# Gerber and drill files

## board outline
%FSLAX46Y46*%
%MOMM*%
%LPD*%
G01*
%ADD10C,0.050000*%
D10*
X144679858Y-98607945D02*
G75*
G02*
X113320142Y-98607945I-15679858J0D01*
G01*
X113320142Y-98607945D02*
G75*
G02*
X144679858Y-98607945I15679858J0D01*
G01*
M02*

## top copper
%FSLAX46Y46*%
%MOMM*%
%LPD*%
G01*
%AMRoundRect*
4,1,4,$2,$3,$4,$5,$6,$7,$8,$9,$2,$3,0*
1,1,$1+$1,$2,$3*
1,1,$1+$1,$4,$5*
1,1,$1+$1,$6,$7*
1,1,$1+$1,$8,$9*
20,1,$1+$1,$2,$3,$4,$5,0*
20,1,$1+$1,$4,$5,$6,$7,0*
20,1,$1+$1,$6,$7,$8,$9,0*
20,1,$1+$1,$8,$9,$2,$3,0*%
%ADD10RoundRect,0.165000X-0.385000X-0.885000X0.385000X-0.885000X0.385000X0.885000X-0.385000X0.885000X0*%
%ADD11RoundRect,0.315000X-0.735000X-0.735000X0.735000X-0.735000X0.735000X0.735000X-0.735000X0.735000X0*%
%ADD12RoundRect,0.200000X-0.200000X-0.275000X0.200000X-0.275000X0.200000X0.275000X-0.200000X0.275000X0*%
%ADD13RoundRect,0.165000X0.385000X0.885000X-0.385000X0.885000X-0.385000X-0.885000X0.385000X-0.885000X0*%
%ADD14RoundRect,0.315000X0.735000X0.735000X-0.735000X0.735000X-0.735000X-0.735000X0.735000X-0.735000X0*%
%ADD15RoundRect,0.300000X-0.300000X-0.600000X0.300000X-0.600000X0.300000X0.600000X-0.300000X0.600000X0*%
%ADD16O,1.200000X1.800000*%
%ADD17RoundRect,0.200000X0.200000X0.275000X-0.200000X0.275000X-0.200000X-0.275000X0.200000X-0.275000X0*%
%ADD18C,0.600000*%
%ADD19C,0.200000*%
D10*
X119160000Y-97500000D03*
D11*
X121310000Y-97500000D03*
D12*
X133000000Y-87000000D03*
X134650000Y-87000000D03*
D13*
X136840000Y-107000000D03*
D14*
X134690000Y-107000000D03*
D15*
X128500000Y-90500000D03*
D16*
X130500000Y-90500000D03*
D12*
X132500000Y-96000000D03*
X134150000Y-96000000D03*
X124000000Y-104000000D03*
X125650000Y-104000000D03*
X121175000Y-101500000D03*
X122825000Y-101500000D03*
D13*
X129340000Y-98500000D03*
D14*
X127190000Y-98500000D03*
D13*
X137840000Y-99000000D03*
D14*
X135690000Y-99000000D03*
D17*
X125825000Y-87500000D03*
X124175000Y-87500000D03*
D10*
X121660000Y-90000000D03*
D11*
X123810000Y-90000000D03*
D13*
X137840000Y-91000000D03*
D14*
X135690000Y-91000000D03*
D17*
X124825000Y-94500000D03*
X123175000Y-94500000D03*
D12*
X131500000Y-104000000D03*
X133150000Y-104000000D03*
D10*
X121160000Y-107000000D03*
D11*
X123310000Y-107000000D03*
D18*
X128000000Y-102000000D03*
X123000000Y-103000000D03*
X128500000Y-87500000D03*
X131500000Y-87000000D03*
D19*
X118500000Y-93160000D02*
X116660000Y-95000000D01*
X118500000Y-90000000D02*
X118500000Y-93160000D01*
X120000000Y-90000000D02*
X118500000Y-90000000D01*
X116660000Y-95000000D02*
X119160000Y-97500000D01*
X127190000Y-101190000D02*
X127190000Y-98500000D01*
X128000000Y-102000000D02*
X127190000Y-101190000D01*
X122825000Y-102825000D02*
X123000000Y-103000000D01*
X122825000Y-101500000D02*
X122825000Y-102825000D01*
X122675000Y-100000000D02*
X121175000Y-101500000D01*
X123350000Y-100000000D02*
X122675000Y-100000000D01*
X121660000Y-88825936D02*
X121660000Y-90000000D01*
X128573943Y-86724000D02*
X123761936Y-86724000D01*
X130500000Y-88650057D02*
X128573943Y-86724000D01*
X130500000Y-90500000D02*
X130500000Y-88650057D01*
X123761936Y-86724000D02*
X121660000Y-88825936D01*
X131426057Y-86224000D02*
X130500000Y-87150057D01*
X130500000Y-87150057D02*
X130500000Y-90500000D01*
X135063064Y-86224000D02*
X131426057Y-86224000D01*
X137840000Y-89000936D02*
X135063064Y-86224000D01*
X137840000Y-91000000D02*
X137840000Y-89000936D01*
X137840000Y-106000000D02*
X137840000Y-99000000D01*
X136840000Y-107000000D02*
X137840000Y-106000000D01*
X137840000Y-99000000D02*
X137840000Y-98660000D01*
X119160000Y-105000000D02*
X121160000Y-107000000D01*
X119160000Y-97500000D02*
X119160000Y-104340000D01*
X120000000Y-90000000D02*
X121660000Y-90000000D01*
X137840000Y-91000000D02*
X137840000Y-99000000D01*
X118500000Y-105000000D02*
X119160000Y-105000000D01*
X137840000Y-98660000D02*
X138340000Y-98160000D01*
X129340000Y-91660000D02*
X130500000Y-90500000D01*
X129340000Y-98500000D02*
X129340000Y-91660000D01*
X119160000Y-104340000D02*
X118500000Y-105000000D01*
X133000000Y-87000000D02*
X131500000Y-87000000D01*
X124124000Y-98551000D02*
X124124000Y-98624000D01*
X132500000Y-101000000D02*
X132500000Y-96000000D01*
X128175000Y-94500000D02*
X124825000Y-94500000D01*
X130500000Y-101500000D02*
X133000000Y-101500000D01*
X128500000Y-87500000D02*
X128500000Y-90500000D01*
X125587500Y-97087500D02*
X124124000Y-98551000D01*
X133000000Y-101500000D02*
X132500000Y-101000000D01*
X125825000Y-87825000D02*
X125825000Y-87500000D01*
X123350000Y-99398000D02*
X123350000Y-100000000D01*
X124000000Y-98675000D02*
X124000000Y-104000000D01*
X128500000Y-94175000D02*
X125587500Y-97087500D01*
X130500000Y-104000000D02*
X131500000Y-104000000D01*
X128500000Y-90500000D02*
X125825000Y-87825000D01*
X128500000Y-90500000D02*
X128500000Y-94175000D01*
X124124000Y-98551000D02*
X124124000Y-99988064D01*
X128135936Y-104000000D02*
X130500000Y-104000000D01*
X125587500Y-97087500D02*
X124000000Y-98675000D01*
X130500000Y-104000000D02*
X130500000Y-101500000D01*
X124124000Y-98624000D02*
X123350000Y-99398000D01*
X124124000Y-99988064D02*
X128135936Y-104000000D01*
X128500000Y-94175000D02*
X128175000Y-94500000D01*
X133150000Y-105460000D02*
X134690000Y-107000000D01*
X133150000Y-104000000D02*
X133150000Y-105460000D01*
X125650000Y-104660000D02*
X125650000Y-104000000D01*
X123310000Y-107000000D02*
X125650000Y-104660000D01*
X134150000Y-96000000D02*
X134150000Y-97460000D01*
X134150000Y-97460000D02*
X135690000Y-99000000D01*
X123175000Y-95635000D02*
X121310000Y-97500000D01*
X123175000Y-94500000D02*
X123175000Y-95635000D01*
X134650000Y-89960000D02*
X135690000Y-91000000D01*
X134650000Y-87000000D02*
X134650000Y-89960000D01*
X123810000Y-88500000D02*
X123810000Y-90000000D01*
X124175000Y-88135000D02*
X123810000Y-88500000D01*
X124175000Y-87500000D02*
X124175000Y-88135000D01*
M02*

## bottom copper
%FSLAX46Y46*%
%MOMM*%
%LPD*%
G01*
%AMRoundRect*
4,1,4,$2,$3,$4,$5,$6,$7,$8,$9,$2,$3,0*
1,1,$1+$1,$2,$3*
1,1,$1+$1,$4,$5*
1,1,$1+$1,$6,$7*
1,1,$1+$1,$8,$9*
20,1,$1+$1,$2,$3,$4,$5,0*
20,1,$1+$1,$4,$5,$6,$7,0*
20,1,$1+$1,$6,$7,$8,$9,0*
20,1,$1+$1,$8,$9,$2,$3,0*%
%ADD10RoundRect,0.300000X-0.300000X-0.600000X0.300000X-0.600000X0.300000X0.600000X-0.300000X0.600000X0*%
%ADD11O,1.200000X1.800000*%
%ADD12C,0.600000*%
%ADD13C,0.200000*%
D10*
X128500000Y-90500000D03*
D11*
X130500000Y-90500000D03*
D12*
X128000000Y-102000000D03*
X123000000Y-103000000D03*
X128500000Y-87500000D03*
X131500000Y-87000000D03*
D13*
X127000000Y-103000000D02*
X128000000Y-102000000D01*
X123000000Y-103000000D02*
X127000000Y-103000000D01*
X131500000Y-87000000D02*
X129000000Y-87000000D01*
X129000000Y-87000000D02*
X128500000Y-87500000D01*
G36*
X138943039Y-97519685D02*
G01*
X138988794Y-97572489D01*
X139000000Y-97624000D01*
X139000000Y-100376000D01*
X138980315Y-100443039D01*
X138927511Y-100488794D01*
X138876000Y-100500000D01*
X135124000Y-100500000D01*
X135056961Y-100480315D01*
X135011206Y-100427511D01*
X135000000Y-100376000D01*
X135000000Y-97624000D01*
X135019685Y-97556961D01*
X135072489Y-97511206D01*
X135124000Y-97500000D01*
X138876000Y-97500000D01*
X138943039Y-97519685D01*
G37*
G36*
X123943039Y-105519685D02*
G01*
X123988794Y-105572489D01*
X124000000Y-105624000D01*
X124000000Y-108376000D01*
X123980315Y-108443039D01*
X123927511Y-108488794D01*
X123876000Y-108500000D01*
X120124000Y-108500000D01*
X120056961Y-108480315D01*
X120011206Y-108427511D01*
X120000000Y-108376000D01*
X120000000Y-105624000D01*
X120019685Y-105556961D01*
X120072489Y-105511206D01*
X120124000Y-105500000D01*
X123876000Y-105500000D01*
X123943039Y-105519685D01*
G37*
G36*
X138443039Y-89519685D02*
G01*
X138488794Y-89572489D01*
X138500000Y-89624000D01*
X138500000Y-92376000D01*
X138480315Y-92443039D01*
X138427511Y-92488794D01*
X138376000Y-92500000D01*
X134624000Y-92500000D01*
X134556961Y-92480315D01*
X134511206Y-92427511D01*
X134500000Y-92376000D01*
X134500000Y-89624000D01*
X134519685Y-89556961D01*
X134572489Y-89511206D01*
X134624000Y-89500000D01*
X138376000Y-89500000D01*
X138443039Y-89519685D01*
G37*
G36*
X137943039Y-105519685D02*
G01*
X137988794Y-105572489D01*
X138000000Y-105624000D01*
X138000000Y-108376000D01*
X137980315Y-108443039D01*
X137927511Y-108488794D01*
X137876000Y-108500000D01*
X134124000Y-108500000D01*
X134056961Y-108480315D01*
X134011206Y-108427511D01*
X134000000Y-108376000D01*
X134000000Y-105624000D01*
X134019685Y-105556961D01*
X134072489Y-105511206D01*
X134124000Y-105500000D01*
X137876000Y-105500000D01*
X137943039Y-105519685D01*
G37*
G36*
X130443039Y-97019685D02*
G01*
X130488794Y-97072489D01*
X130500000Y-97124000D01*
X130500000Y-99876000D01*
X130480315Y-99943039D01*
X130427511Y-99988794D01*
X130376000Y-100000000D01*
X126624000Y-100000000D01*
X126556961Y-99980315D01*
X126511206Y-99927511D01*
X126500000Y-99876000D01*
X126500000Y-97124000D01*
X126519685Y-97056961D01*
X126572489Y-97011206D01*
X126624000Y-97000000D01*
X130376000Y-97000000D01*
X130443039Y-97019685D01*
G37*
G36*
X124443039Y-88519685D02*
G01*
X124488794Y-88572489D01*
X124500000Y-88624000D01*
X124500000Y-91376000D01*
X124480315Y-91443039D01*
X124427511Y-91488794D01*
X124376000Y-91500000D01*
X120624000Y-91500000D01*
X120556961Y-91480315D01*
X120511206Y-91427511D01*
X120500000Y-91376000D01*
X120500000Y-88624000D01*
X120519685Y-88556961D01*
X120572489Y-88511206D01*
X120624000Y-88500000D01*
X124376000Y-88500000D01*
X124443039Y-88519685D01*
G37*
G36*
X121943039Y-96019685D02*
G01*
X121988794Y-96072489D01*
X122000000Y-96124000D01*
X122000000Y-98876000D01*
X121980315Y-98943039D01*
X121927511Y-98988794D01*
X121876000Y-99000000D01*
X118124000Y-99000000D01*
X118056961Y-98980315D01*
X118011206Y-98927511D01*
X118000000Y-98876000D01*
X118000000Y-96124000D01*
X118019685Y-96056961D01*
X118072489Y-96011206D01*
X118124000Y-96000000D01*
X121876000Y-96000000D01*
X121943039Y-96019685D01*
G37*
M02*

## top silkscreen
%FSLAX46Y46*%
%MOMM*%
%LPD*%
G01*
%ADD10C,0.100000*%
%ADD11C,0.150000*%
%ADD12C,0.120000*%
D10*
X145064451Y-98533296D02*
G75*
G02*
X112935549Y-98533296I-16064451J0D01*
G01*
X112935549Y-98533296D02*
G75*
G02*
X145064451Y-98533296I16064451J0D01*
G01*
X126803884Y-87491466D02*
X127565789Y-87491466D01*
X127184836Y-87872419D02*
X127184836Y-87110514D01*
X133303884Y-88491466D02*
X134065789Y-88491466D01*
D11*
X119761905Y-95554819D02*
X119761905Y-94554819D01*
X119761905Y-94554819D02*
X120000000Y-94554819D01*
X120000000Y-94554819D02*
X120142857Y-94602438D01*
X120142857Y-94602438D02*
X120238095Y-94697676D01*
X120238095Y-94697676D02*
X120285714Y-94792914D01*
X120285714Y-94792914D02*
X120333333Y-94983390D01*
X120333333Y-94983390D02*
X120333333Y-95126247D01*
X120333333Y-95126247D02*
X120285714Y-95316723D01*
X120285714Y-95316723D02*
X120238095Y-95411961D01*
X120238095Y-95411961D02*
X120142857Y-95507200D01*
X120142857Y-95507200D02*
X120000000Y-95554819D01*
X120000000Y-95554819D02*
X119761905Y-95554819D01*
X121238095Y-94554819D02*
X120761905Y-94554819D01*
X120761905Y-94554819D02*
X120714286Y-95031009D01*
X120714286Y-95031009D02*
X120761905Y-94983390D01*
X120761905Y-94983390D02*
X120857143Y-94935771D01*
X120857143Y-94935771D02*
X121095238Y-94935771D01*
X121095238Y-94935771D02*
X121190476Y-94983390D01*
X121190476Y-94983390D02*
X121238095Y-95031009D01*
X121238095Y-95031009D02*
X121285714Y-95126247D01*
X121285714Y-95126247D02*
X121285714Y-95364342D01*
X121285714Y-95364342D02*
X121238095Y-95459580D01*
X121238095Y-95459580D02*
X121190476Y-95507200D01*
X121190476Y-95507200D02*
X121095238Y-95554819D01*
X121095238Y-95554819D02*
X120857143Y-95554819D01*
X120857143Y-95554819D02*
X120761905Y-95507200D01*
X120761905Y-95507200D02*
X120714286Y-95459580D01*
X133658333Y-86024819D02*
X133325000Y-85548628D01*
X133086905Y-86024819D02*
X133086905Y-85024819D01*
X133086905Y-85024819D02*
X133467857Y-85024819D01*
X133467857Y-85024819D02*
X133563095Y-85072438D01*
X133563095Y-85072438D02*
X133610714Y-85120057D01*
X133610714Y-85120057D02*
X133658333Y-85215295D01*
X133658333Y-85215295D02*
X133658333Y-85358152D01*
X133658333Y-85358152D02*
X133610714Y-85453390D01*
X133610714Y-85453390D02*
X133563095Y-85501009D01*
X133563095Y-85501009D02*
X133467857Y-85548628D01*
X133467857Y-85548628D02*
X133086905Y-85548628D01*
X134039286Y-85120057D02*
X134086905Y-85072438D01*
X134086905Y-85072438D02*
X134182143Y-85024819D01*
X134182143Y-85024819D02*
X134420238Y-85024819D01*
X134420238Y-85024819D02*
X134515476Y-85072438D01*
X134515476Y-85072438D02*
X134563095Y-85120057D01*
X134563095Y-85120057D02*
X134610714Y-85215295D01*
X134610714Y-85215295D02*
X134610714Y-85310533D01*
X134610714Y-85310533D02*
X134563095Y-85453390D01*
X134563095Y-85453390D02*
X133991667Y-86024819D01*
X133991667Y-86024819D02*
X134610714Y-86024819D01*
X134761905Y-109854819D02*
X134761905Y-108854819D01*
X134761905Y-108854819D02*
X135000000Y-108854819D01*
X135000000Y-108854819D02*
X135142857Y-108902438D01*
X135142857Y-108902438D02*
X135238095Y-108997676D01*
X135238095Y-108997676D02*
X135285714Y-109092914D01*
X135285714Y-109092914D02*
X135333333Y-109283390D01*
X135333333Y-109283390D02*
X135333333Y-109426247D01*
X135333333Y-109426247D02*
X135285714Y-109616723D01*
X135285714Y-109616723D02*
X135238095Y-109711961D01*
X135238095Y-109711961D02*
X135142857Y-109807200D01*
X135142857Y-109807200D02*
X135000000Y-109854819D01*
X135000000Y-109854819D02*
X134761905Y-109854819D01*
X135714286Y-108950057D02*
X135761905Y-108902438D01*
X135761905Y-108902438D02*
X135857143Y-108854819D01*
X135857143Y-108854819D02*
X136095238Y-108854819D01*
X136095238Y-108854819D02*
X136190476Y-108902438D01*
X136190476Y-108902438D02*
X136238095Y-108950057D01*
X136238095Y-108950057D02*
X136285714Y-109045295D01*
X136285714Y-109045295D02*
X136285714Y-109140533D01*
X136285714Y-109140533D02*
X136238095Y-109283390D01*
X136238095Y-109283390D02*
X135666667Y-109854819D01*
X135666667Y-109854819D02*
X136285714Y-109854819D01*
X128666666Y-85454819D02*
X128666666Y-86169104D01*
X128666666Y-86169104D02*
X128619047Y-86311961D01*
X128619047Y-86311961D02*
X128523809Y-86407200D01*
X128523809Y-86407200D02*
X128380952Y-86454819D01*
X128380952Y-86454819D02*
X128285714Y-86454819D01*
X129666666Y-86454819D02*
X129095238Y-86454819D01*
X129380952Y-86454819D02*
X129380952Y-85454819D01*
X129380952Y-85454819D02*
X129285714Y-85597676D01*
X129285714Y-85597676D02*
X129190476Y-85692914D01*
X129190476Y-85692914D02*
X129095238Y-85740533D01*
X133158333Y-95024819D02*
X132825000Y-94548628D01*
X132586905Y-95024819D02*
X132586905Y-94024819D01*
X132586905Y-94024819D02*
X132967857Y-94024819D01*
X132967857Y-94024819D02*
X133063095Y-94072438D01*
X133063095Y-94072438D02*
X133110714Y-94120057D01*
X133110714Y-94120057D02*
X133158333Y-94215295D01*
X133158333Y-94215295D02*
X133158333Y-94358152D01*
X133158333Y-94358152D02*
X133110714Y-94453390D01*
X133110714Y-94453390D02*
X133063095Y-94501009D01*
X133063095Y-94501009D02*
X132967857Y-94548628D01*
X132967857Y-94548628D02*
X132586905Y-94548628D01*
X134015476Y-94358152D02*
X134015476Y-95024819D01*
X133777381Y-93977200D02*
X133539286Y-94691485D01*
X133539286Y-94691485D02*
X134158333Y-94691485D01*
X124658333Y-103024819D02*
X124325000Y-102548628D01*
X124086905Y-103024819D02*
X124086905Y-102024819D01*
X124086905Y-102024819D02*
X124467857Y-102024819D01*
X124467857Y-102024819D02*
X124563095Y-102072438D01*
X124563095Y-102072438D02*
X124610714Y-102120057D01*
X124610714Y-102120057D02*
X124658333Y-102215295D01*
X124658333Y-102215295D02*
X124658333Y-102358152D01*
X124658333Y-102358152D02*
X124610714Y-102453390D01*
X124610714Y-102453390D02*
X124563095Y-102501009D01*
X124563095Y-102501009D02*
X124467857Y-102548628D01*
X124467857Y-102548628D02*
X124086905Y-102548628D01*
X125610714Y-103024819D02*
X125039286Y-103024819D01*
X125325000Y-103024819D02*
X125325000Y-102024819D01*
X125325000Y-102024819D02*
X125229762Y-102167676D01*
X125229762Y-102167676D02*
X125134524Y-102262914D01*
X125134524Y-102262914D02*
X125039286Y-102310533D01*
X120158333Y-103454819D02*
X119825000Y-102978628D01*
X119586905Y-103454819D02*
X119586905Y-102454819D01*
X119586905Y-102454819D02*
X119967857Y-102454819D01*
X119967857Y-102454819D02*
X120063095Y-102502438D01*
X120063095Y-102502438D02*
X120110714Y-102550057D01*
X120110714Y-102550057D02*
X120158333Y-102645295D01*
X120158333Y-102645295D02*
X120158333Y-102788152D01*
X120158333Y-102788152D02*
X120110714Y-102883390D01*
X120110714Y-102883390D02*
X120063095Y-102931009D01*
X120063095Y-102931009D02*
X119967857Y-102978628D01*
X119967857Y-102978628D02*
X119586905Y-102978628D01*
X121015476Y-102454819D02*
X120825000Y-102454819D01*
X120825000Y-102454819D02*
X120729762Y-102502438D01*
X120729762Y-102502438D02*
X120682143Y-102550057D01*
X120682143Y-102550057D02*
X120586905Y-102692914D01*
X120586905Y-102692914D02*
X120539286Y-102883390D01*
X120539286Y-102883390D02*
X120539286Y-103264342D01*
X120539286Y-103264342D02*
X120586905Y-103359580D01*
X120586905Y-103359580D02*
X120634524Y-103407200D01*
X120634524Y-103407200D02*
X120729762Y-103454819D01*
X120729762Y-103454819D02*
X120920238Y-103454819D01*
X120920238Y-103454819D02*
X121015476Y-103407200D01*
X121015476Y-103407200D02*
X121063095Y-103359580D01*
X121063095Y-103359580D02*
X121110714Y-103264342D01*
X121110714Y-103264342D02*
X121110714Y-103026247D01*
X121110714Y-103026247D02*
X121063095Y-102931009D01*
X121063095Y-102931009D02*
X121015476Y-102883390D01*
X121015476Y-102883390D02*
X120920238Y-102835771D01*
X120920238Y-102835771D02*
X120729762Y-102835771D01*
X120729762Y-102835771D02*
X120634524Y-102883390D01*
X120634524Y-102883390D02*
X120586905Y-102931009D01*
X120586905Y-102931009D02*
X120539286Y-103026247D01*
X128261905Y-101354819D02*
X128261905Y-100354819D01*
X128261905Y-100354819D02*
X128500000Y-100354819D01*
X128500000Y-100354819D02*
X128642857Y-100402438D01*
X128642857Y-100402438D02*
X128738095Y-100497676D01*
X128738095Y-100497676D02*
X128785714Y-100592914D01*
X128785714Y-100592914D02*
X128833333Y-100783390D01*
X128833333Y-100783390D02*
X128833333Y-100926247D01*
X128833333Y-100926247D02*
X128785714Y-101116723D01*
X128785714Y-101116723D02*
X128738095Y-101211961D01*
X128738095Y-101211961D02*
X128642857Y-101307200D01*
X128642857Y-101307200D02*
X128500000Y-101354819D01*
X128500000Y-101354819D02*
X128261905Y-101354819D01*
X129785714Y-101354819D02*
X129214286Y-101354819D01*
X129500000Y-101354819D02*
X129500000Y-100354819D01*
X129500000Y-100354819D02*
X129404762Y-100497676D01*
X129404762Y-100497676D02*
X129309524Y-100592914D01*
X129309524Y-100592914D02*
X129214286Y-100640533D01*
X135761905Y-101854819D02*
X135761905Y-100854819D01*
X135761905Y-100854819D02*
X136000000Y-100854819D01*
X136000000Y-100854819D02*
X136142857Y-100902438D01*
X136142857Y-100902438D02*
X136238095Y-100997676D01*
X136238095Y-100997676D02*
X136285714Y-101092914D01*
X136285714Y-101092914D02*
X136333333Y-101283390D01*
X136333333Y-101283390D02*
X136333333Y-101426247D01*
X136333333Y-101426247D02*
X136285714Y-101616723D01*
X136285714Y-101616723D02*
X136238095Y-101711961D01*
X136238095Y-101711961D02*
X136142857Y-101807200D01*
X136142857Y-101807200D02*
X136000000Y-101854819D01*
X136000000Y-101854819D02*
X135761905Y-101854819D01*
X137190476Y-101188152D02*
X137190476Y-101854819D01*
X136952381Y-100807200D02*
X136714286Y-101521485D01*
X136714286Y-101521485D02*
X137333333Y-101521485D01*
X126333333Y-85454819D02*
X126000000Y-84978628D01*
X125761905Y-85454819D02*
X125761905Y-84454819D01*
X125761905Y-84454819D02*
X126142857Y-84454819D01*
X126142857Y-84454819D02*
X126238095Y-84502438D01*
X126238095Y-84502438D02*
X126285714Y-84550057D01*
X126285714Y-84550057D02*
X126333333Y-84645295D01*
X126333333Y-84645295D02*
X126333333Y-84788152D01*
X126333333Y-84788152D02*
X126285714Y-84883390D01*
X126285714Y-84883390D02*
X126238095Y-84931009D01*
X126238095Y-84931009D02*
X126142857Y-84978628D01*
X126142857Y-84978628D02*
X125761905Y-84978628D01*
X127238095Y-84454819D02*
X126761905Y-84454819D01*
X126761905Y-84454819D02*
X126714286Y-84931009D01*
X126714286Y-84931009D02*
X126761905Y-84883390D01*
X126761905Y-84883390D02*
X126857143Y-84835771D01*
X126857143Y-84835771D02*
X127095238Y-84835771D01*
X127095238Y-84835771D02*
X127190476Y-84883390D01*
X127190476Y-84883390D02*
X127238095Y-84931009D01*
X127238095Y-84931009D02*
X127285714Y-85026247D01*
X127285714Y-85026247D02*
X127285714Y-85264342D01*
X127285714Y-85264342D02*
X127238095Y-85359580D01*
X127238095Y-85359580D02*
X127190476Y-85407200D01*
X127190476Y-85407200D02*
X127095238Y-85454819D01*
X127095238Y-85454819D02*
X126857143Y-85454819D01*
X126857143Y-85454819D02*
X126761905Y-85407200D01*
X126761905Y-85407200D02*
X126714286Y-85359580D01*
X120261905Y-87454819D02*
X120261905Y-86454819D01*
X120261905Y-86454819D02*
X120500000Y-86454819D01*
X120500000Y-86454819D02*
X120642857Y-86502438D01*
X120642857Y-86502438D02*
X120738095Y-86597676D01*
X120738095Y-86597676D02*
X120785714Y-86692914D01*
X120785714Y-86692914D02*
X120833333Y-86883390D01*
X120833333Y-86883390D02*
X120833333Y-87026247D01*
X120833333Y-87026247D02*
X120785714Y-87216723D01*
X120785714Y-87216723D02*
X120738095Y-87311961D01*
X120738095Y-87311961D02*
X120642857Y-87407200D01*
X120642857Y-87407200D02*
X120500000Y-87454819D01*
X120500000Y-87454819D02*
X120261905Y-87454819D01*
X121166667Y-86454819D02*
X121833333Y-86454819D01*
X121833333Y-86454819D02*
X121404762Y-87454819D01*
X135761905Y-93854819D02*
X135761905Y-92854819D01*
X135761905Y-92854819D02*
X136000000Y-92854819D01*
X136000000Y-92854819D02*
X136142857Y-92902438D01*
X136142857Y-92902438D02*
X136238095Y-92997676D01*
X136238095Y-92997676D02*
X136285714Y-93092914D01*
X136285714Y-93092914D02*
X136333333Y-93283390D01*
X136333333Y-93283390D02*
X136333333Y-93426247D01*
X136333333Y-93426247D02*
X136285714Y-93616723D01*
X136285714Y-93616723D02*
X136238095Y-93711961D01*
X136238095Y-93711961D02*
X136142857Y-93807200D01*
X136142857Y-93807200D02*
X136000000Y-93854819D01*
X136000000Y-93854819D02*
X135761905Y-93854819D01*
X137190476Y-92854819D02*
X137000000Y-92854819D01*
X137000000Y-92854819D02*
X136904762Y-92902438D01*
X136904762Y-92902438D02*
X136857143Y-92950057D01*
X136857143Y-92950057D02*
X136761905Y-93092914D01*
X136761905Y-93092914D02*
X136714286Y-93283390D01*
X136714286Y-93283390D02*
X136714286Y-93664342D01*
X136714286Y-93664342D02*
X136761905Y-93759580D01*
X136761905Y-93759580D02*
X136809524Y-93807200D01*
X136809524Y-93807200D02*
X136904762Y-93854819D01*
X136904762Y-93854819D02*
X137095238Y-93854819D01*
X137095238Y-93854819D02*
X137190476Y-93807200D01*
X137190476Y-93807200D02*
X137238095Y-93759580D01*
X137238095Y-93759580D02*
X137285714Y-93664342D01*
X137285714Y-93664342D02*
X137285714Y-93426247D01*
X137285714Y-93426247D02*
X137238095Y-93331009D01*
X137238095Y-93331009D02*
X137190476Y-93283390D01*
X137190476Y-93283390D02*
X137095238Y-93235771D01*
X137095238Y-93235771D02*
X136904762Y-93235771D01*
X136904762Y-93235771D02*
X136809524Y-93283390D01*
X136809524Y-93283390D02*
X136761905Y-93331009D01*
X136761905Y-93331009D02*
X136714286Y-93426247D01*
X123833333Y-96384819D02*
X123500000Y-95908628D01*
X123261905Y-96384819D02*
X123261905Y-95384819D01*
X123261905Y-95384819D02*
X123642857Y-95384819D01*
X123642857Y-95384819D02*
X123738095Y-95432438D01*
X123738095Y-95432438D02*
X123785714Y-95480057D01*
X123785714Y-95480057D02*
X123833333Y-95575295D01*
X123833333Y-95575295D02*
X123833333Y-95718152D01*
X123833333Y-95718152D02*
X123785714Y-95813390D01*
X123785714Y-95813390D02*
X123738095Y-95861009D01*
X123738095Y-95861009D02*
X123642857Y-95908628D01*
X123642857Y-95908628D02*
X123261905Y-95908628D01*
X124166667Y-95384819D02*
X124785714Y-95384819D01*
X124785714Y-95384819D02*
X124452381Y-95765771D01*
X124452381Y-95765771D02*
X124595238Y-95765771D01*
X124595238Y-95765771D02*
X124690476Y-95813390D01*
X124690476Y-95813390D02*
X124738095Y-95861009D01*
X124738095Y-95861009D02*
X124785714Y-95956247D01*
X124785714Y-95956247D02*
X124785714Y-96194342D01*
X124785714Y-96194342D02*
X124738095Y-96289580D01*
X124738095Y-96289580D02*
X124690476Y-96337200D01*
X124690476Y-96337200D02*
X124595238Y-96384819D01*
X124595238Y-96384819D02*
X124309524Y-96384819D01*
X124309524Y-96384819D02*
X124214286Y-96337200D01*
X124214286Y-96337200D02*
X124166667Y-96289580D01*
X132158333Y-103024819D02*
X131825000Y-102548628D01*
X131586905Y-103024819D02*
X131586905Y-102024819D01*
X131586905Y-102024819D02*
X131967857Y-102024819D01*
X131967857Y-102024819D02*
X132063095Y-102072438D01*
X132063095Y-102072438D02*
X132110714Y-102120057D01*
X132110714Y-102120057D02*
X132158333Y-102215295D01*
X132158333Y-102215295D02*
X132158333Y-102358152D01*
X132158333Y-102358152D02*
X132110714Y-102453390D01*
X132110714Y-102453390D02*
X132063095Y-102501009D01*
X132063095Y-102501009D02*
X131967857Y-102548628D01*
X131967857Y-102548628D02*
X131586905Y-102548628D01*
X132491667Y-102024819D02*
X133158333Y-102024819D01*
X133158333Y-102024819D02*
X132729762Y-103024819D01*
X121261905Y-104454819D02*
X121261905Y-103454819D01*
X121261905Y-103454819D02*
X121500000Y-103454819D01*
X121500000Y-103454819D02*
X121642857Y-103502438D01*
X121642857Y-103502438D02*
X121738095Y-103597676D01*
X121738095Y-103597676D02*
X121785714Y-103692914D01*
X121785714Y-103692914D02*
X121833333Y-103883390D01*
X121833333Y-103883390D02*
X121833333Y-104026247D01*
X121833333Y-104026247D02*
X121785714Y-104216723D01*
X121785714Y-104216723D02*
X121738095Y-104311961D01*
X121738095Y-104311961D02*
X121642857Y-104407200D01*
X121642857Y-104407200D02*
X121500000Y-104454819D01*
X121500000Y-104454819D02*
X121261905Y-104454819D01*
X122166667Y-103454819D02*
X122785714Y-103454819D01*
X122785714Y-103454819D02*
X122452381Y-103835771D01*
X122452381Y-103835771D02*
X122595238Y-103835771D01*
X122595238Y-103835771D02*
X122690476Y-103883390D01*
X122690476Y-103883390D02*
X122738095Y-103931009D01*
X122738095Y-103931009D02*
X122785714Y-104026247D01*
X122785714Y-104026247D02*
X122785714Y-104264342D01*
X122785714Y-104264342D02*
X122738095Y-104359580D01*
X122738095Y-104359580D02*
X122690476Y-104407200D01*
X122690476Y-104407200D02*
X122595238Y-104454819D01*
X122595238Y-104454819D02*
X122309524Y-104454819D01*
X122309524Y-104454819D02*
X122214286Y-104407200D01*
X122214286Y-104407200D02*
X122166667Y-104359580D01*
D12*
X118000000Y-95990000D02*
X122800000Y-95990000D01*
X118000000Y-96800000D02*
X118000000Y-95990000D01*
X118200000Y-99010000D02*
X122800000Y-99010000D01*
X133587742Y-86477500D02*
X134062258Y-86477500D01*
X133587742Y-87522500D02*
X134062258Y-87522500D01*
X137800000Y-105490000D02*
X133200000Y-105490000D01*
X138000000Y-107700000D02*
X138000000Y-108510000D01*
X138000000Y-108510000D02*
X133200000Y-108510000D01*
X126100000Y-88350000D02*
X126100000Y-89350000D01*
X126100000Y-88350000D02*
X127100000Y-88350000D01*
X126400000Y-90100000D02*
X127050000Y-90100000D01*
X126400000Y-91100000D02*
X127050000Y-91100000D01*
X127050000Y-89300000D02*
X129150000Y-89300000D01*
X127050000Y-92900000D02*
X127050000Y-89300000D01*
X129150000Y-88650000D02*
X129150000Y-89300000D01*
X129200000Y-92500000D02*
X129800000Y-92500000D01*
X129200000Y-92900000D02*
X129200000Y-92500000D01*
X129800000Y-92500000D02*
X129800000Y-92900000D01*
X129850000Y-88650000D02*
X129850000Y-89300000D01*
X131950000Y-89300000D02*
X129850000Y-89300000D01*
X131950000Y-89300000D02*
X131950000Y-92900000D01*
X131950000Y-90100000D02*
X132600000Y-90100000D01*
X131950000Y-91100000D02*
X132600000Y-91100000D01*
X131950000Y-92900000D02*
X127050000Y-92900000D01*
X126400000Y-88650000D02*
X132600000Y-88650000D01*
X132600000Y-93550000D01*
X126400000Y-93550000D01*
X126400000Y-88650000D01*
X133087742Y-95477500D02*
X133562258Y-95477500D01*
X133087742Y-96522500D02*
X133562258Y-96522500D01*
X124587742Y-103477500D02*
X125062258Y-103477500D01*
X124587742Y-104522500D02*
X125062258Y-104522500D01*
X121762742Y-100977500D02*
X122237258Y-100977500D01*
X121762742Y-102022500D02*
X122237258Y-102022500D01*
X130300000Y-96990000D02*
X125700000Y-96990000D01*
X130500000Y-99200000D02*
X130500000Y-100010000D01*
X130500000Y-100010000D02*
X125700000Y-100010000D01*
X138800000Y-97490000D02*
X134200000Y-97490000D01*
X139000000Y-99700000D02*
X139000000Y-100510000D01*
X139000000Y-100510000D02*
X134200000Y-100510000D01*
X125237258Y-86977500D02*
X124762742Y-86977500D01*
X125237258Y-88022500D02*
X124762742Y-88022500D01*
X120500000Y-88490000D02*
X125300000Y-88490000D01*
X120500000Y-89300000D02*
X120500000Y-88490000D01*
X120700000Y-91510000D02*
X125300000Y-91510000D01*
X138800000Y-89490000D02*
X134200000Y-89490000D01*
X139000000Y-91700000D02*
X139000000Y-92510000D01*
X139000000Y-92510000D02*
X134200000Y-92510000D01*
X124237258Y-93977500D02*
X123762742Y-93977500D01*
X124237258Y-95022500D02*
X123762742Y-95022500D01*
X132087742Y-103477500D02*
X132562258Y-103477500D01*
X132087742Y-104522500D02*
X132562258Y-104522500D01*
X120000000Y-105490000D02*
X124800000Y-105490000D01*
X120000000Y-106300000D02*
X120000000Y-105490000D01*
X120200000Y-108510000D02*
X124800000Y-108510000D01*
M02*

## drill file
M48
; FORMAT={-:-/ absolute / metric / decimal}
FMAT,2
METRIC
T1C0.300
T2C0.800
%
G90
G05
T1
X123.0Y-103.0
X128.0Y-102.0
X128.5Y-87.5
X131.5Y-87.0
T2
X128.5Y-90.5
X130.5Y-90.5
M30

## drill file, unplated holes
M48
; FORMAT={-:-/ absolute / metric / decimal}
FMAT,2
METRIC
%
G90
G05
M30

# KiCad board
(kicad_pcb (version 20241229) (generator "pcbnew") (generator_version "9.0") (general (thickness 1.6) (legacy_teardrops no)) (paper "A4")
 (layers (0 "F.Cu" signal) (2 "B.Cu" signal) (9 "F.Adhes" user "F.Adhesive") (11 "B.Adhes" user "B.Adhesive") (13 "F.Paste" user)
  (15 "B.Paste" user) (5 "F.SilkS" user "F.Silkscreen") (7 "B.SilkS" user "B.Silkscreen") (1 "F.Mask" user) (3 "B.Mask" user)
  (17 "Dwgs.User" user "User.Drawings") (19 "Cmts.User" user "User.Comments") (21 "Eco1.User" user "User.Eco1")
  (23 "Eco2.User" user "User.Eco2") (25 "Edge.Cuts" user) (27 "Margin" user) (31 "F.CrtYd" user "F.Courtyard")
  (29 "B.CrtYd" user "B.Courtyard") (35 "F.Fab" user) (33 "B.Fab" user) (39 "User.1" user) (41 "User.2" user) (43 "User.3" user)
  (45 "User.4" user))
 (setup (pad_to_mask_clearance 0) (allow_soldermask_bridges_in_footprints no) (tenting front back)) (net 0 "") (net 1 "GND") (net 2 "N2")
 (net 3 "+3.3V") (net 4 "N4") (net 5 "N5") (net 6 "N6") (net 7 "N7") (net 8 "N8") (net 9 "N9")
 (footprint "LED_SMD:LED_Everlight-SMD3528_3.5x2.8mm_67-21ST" (layer "F.Cu") (at 120.5 97.5)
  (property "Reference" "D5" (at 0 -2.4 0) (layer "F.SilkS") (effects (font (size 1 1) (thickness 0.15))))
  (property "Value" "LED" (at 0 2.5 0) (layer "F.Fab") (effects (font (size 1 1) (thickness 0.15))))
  (fp_line (start -2.5 -1.51) (end 2.3 -1.51) (stroke (width 0.12) (type solid)) (layer "F.SilkS"))
  (fp_line (start -2.5 -0.7) (end -2.5 -1.51) (stroke (width 0.12) (type solid)) (layer "F.SilkS"))
  (fp_line (start -2.3 1.51) (end 2.3 1.51) (stroke (width 0.12) (type solid)) (layer "F.SilkS"))
  (pad "1" smd roundrect (at -1.34 0) (size 1.1 2.1) (layers "F.Cu" "F.Mask" "F.Paste") (roundrect_rratio 0.15) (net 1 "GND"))
  (pad "2" smd roundrect (at 0.81 0) (size 2.1 2.1) (layers "F.Cu" "F.Mask" "F.Paste") (roundrect_rratio 0.15) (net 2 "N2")))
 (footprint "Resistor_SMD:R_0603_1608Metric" (layer "F.Cu") (at 133.825 87)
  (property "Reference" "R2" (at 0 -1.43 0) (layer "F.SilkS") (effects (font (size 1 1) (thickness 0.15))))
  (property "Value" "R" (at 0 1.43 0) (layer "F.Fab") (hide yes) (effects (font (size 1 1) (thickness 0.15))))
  (fp_line (start -0.237258 -0.5225) (end 0.237258 -0.5225) (stroke (width 0.12) (type solid)) (layer "F.SilkS"))
  (fp_line (start -0.237258 0.5225) (end 0.237258 0.5225) (stroke (width 0.12) (type solid)) (layer "F.SilkS"))
  (pad "1" smd roundrect (at -0.825 0) (size 0.8 0.95) (layers "F.Cu" "F.Mask" "F.Paste") (roundrect_rratio 0.25) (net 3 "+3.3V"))
  (pad "2" smd roundrect (at 0.825 0) (size 0.8 0.95) (layers "F.Cu" "F.Mask" "F.Paste") (roundrect_rratio 0.25) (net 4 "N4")))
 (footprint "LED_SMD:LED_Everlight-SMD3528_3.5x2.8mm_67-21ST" (layer "F.Cu") (at 135.5 107 180)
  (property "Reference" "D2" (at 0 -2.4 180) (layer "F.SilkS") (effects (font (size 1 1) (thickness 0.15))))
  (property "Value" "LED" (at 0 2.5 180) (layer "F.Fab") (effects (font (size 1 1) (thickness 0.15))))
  (fp_line (start -2.3 1.51) (end 2.3 1.51) (stroke (width 0.12) (type solid)) (layer "F.SilkS"))
  (fp_line (start -2.5 -0.7) (end -2.5 -1.51) (stroke (width 0.12) (type solid)) (layer "F.SilkS"))
  (fp_line (start -2.5 -1.51) (end 2.3 -1.51) (stroke (width 0.12) (type solid)) (layer "F.SilkS"))
  (pad "1" smd roundrect (at -1.34 0 180) (size 1.1 2.1) (layers "F.Cu" "F.Mask" "F.Paste") (roundrect_rratio 0.15) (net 1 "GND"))
  (pad "2" smd roundrect (at 0.81 0 180) (size 2.1 2.1) (layers "F.Cu" "F.Mask" "F.Paste") (roundrect_rratio 0.15) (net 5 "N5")))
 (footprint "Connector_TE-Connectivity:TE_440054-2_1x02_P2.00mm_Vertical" (layer "F.Cu") (at 128.5 90.5)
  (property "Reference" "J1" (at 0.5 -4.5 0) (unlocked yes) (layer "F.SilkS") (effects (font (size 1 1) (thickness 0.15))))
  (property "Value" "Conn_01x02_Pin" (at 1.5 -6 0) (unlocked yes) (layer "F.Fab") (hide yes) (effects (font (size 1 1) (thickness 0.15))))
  (fp_line (start -2.4 -2.15) (end -2.4 -1.15) (stroke (width 0.12) (type solid)) (layer "F.SilkS"))
  (fp_line (start -2.4 -2.15) (end -1.4 -2.15) (stroke (width 0.12) (type solid)) (layer "F.SilkS"))
  (fp_line (start -2.1 -0.4) (end -1.45 -0.4) (stroke (width 0.12) (type solid)) (layer "F.SilkS"))
  (fp_line (start -2.1 0.6) (end -1.45 0.6) (stroke (width 0.12) (type solid)) (layer "F.SilkS"))
  (fp_line (start -1.45 -1.2) (end 0.65 -1.2) (stroke (width 0.12) (type solid)) (layer "F.SilkS"))
  (fp_line (start -1.45 2.4) (end -1.45 -1.2) (stroke (width 0.12) (type solid)) (layer "F.SilkS"))
  (fp_line (start 0.65 -1.85) (end 0.65 -1.2) (stroke (width 0.12) (type solid)) (layer "F.SilkS"))
  (fp_line (start 0.7 2) (end 1.3 2) (stroke (width 0.12) (type solid)) (layer "F.SilkS"))
  (fp_line (start 0.7 2.4) (end 0.7 2) (stroke (width 0.12) (type solid)) (layer "F.SilkS"))
  (fp_line (start 1.3 2) (end 1.3 2.4) (stroke (width 0.12) (type solid)) (layer "F.SilkS"))
  (fp_line (start 1.35 -1.85) (end 1.35 -1.2) (stroke (width 0.12) (type solid)) (layer "F.SilkS"))
  (fp_line (start 3.45 -1.2) (end 1.35 -1.2) (stroke (width 0.12) (type solid)) (layer "F.SilkS"))
  (fp_line (start 3.45 -1.2) (end 3.45 2.4) (stroke (width 0.12) (type solid)) (layer "F.SilkS"))
  (fp_line (start 3.45 -0.4) (end 4.1 -0.4) (stroke (width 0.12) (type solid)) (layer "F.SilkS"))
  (fp_line (start 3.45 0.6) (end 4.1 0.6) (stroke (width 0.12) (type solid)) (layer "F.SilkS"))
  (fp_line (start 3.45 2.4) (end -1.45 2.4) (stroke (width 0.12) (type solid)) (layer "F.SilkS"))
  (fp_rect (start -2.1 -1.85) (end 4.1 3.05) (stroke (width 0.12) (type solid)) (fill no) (layer "F.SilkS"))
  (pad "1" thru_hole roundrect (at 0 0) (size 1.2 1.8) (drill 0.8) (layers "*.Cu" "*.Mask") (remove_unused_layers no)
   (roundrect_rratio 0.25) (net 3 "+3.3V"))
  (pad "2" thru_hole oval (at 2 0) (size 1.2 1.8) (drill 0.8) (layers "*.Cu" "*.Mask") (remove_unused_layers no) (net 1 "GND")))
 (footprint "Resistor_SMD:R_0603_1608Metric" (layer "F.Cu") (at 133.325 96)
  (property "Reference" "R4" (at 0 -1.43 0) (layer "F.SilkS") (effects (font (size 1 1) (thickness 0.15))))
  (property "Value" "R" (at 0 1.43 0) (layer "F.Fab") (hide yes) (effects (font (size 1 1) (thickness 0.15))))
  (fp_line (start -0.237258 -0.5225) (end 0.237258 -0.5225) (stroke (width 0.12) (type solid)) (layer "F.SilkS"))
  (fp_line (start -0.237258 0.5225) (end 0.237258 0.5225) (stroke (width 0.12) (type solid)) (layer "F.SilkS"))
  (pad "1" smd roundrect (at -0.825 0) (size 0.8 0.95) (layers "F.Cu" "F.Mask" "F.Paste") (roundrect_rratio 0.25) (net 3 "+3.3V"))
  (pad "2" smd roundrect (at 0.825 0) (size 0.8 0.95) (layers "F.Cu" "F.Mask" "F.Paste") (roundrect_rratio 0.25) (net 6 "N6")))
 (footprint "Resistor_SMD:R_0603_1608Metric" (layer "F.Cu") (at 124.825 104)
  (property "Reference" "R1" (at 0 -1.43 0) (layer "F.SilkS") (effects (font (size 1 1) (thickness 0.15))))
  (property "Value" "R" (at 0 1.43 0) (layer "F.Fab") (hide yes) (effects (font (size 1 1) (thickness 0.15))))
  (fp_line (start -0.237258 -0.5225) (end 0.237258 -0.5225) (stroke (width 0.12) (type solid)) (layer "F.SilkS"))
  (fp_line (start -0.237258 0.5225) (end 0.237258 0.5225) (stroke (width 0.12) (type solid)) (layer "F.SilkS"))
  (pad "1" smd roundrect (at -0.825 0) (size 0.8 0.95) (layers "F.Cu" "F.Mask" "F.Paste") (roundrect_rratio 0.25) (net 3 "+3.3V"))
  (pad "2" smd roundrect (at 0.825 0) (size 0.8 0.95) (layers "F.Cu" "F.Mask" "F.Paste") (roundrect_rratio 0.25) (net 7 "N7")))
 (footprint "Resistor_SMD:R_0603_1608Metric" (layer "F.Cu") (at 122 101.5)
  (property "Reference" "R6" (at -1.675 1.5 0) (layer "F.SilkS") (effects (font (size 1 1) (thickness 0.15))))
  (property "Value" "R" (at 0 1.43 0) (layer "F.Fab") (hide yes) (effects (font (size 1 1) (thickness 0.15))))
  (fp_line (start -0.237258 -0.5225) (end 0.237258 -0.5225) (stroke (width 0.12) (type solid)) (layer "F.SilkS"))
  (fp_line (start -0.237258 0.5225) (end 0.237258 0.5225) (stroke (width 0.12) (type solid)) (layer "F.SilkS"))
  (pad "1" smd roundrect (at -0.825 0) (size 0.8 0.95) (layers "F.Cu" "F.Mask" "F.Paste") (roundrect_rratio 0.25) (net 3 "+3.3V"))
  (pad "2" smd roundrect (at 0.825 0) (size 0.8 0.95) (layers "F.Cu" "F.Mask" "F.Paste") (roundrect_rratio 0.25) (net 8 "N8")))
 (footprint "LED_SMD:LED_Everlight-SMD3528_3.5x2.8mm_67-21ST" (layer "F.Cu") (at 128 98.5 180)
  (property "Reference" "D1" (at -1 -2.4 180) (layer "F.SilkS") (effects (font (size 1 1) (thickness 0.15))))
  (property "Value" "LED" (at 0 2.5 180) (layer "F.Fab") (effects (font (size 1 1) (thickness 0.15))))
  (fp_line (start -2.3 1.51) (end 2.3 1.51) (stroke (width 0.12) (type solid)) (layer "F.SilkS"))
  (fp_line (start -2.5 -0.7) (end -2.5 -1.51) (stroke (width 0.12) (type solid)) (layer "F.SilkS"))
  (fp_line (start -2.5 -1.51) (end 2.3 -1.51) (stroke (width 0.12) (type solid)) (layer "F.SilkS"))
  (pad "1" smd roundrect (at -1.34 0 180) (size 1.1 2.1) (layers "F.Cu" "F.Mask" "F.Paste") (roundrect_rratio 0.15) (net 1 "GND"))
  (pad "2" smd roundrect (at 0.81 0 180) (size 2.1 2.1) (layers "F.Cu" "F.Mask" "F.Paste") (roundrect_rratio 0.15) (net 8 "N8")))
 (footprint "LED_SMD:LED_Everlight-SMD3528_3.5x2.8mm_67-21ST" (layer "F.Cu") (at 136.5 99 180)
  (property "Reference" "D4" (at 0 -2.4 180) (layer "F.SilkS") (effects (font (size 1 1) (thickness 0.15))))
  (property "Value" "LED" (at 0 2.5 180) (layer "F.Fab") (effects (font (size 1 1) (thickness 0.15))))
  (fp_line (start -2.3 1.51) (end 2.3 1.51) (stroke (width 0.12) (type solid)) (layer "F.SilkS"))
  (fp_line (start -2.5 -0.7) (end -2.5 -1.51) (stroke (width 0.12) (type solid)) (layer "F.SilkS"))
  (fp_line (start -2.5 -1.51) (end 2.3 -1.51) (stroke (width 0.12) (type solid)) (layer "F.SilkS"))
  (pad "1" smd roundrect (at -1.34 0 180) (size 1.1 2.1) (layers "F.Cu" "F.Mask" "F.Paste") (roundrect_rratio 0.15) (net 1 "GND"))
  (pad "2" smd roundrect (at 0.81 0 180) (size 2.1 2.1) (layers "F.Cu" "F.Mask" "F.Paste") (roundrect_rratio 0.15) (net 6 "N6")))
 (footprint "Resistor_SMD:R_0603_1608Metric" (layer "F.Cu") (at 125 87.5 180)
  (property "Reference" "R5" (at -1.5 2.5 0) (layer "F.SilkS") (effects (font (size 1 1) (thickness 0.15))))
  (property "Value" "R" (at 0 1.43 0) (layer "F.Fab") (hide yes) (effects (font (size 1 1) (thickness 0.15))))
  (fp_line (start -0.237258 0.5225) (end 0.237258 0.5225) (stroke (width 0.12) (type solid)) (layer "F.SilkS"))
  (fp_line (start -0.237258 -0.5225) (end 0.237258 -0.5225) (stroke (width 0.12) (type solid)) (layer "F.SilkS"))
  (pad "1" smd roundrect (at -0.825 0 180) (size 0.8 0.95) (layers "F.Cu" "F.Mask" "F.Paste") (roundrect_rratio 0.25) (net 3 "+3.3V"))
  (pad "2" smd roundrect (at 0.825 0 180) (size 0.8 0.95) (layers "F.Cu" "F.Mask" "F.Paste") (roundrect_rratio 0.25) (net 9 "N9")))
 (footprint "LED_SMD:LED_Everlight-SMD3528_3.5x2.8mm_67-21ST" (layer "F.Cu") (at 123 90)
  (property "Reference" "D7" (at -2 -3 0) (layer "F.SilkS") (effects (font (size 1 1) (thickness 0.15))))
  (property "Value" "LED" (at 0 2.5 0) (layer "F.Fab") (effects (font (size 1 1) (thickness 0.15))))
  (fp_line (start -2.5 -1.51) (end 2.3 -1.51) (stroke (width 0.12) (type solid)) (layer "F.SilkS"))
  (fp_line (start -2.5 -0.7) (end -2.5 -1.51) (stroke (width 0.12) (type solid)) (layer "F.SilkS"))
  (fp_line (start -2.3 1.51) (end 2.3 1.51) (stroke (width 0.12) (type solid)) (layer "F.SilkS"))
  (pad "1" smd roundrect (at -1.34 0) (size 1.1 2.1) (layers "F.Cu" "F.Mask" "F.Paste") (roundrect_rratio 0.15) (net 1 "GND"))
  (pad "2" smd roundrect (at 0.81 0) (size 2.1 2.1) (layers "F.Cu" "F.Mask" "F.Paste") (roundrect_rratio 0.15) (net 9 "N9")))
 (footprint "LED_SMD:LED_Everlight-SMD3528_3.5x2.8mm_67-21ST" (layer "F.Cu") (at 136.5 91 180)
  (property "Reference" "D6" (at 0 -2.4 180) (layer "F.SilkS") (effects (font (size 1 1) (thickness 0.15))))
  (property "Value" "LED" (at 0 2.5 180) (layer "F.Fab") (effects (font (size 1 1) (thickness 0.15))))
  (fp_line (start -2.3 1.51) (end 2.3 1.51) (stroke (width 0.12) (type solid)) (layer "F.SilkS"))
  (fp_line (start -2.5 -0.7) (end -2.5 -1.51) (stroke (width 0.12) (type solid)) (layer "F.SilkS"))
  (fp_line (start -2.5 -1.51) (end 2.3 -1.51) (stroke (width 0.12) (type solid)) (layer "F.SilkS"))
  (pad "1" smd roundrect (at -1.34 0 180) (size 1.1 2.1) (layers "F.Cu" "F.Mask" "F.Paste") (roundrect_rratio 0.15) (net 1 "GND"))
  (pad "2" smd roundrect (at 0.81 0 180) (size 2.1 2.1) (layers "F.Cu" "F.Mask" "F.Paste") (roundrect_rratio 0.15) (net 4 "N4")))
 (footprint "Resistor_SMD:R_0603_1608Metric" (layer "F.Cu") (at 124 94.5 180)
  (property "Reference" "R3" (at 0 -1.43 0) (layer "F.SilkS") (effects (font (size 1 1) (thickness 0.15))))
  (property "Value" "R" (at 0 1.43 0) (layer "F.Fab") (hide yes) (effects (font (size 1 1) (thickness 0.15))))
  (fp_line (start -0.237258 0.5225) (end 0.237258 0.5225) (stroke (width 0.12) (type solid)) (layer "F.SilkS"))
  (fp_line (start -0.237258 -0.5225) (end 0.237258 -0.5225) (stroke (width 0.12) (type solid)) (layer "F.SilkS"))
  (pad "1" smd roundrect (at -0.825 0 180) (size 0.8 0.95) (layers "F.Cu" "F.Mask" "F.Paste") (roundrect_rratio 0.25) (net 3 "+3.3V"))
  (pad "2" smd roundrect (at 0.825 0 180) (size 0.8 0.95) (layers "F.Cu" "F.Mask" "F.Paste") (roundrect_rratio 0.25) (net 2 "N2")))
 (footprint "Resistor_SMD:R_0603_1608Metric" (layer "F.Cu") (at 132.325 104)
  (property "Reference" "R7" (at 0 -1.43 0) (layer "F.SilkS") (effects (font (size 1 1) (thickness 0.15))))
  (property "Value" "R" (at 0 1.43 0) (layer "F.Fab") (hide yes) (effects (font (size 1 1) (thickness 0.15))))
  (fp_line (start -0.237258 -0.5225) (end 0.237258 -0.5225) (stroke (width 0.12) (type solid)) (layer "F.SilkS"))
  (fp_line (start -0.237258 0.5225) (end 0.237258 0.5225) (stroke (width 0.12) (type solid)) (layer "F.SilkS"))
  (pad "1" smd roundrect (at -0.825 0) (size 0.8 0.95) (layers "F.Cu" "F.Mask" "F.Paste") (roundrect_rratio 0.25) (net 3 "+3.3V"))
  (pad "2" smd roundrect (at 0.825 0) (size 0.8 0.95) (layers "F.Cu" "F.Mask" "F.Paste") (roundrect_rratio 0.25) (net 5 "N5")))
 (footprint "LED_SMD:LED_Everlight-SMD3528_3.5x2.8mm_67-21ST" (layer "F.Cu") (at 122.5 107)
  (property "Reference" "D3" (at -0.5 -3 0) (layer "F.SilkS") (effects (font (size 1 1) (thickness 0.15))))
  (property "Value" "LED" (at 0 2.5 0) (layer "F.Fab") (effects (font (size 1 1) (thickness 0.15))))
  (fp_line (start -2.5 -1.51) (end 2.3 -1.51) (stroke (width 0.12) (type solid)) (layer "F.SilkS"))
  (fp_line (start -2.5 -0.7) (end -2.5 -1.51) (stroke (width 0.12) (type solid)) (layer "F.SilkS"))
  (fp_line (start -2.3 1.51) (end 2.3 1.51) (stroke (width 0.12) (type solid)) (layer "F.SilkS"))
  (pad "1" smd roundrect (at -1.34 0) (size 1.1 2.1) (layers "F.Cu" "F.Mask" "F.Paste") (roundrect_rratio 0.15) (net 1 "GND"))
  (pad "2" smd roundrect (at 0.81 0) (size 2.1 2.1) (layers "F.Cu" "F.Mask" "F.Paste") (roundrect_rratio 0.15) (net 7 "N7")))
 (gr_circle (center 129 98.533296) (end 128 82.5) (stroke (width 0.1) (type solid)) (fill no) (layer "F.SilkS"))
 (gr_circle (center 129 98.607945) (end 130.5 83) (stroke (width 0.05) (type default)) (fill no) (layer "Edge.Cuts"))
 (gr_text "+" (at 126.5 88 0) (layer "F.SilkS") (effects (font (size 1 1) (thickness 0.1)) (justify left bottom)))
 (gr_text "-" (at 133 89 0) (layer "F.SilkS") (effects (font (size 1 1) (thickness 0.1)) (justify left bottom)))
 (segment (start 137.84 99) (end 137.84 98.66) (width 0.2) (layer "F.Cu") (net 1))
 (segment (start 137.84 89.000936) (end 135.063064 86.224) (width 0.2) (layer "F.Cu") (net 1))
 (segment (start 120 90) (end 118.5 90) (width 0.2) (layer "F.Cu") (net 1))
 (segment (start 119.16 105) (end 121.16 107) (width 0.2) (layer "F.Cu") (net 1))
 (segment (start 119.16 97.5) (end 119.16 104.34) (width 0.2) (layer "F.Cu") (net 1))
 (segment (start 130.5 87.150057) (end 130.5 90.5) (width 0.2) (layer "F.Cu") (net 1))
 (segment (start 120 90) (end 121.66 90) (width 0.2) (layer "F.Cu") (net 1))
 (segment (start 135.063064 86.224) (end 131.426057 86.224) (width 0.2) (layer "F.Cu") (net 1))
 (segment (start 136.84 107) (end 137.84 106) (width 0.2) (layer "F.Cu") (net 1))
 (segment (start 130.5 88.650057) (end 128.573943 86.724) (width 0.2) (layer "F.Cu") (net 1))
 (segment (start 137.84 91) (end 137.84 99) (width 0.2) (layer "F.Cu") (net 1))
 (segment (start 137.84 91) (end 137.84 89.000936) (width 0.2) (layer "F.Cu") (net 1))
 (segment (start 116.66 95) (end 119.16 97.5) (width 0.2) (layer "F.Cu") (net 1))
 (segment (start 118.5 105) (end 119.16 105) (width 0.2) (layer "F.Cu") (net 1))
 (segment (start 137.84 106) (end 137.84 99) (width 0.2) (layer "F.Cu") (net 1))
 (segment (start 121.66 88.825936) (end 121.66 90) (width 0.2) (layer "F.Cu") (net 1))
 (segment (start 130.5 90.5) (end 130.5 88.650057) (width 0.2) (layer "F.Cu") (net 1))
 (segment (start 128.573943 86.724) (end 123.761936 86.724) (width 0.2) (layer "F.Cu") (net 1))
 (segment (start 137.84 98.66) (end 138.34 98.16) (width 0.2) (layer "F.Cu") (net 1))
 (segment (start 129.34 91.66) (end 130.5 90.5) (width 0.2) (layer "F.Cu") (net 1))
 (segment (start 131.426057 86.224) (end 130.5 87.150057) (width 0.2) (layer "F.Cu") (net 1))
 (segment (start 118.5 90) (end 118.5 93.16) (width 0.2) (layer "F.Cu") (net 1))
 (segment (start 123.761936 86.724) (end 121.66 88.825936) (width 0.2) (layer "F.Cu") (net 1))
 (segment (start 129.34 98.5) (end 129.34 91.66) (width 0.2) (layer "F.Cu") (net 1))
 (segment (start 119.16 104.34) (end 118.5 105) (width 0.2) (layer "F.Cu") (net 1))
 (segment (start 118.5 93.16) (end 116.66 95) (width 0.2) (layer "F.Cu") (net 1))
 (segment (start 122.675 100) (end 121.175 101.5) (width 0.2) (layer "F.Cu") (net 3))
 (segment (start 133 87) (end 131.5 87) (width 0.2) (layer "F.Cu") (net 3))
 (segment (start 124.124 98.551) (end 124.124 98.624) (width 0.2) (layer "F.Cu") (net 3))
 (segment (start 132.5 101) (end 132.5 96) (width 0.2) (layer "F.Cu") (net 3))
 (segment (start 128.175 94.5) (end 124.825 94.5) (width 0.2) (layer "F.Cu") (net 3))
 (segment (start 130.5 101.5) (end 133 101.5) (width 0.2) (layer "F.Cu") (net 3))
 (segment (start 128.5 87.5) (end 128.5 90.5) (width 0.2) (layer "F.Cu") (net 3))
 (segment (start 125.5875 97.0875) (end 124.124 98.551) (width 0.2) (layer "F.Cu") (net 3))
 (segment (start 133 101.5) (end 132.5 101) (width 0.2) (layer "F.Cu") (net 3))
 (segment (start 125.825 87.825) (end 125.825 87.5) (width 0.2) (layer "F.Cu") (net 3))
 (segment (start 123.35 99.398) (end 123.35 100) (width 0.2) (layer "F.Cu") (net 3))
 (segment (start 124 98.675) (end 124 104) (width 0.2) (layer "F.Cu") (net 3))
 (segment (start 128.5 94.175) (end 125.5875 97.0875) (width 0.2) (layer "F.Cu") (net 3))
 (segment (start 130.5 104) (end 131.5 104) (width 0.2) (layer "F.Cu") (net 3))
 (segment (start 128.5 90.5) (end 125.825 87.825) (width 0.2) (layer "F.Cu") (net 3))
 (segment (start 123.35 100) (end 122.675 100) (width 0.2) (layer "F.Cu") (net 3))
 (segment (start 128.5 90.5) (end 128.5 94.175) (width 0.2) (layer "F.Cu") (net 3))
 (segment (start 124.124 98.551) (end 124.124 99.988064) (width 0.2) (layer "F.Cu") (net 3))
 (segment (start 128.135936 104) (end 130.5 104) (width 0.2) (layer "F.Cu") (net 3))
 (segment (start 125.5875 97.0875) (end 124 98.675) (width 0.2) (layer "F.Cu") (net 3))
 (segment (start 130.5 104) (end 130.5 101.5) (width 0.2) (layer "F.Cu") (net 3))
 (segment (start 124.124 98.624) (end 123.35 99.398) (width 0.2) (layer "F.Cu") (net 3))
 (segment (start 124.124 99.988064) (end 128.135936 104) (width 0.2) (layer "F.Cu") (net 3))
 (segment (start 128.5 94.175) (end 128.175 94.5) (width 0.2) (layer "F.Cu") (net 3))
 (via (at 128.5 87.5) (size 0.6) (drill 0.3) (layers "F.Cu" "B.Cu") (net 3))
 (via (at 131.5 87) (size 0.6) (drill 0.3) (layers "F.Cu" "B.Cu") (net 3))
 (segment (start 131.5 87) (end 129 87) (width 0.2) (layer "B.Cu") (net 3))
 (segment (start 129 87) (end 128.5 87.5) (width 0.2) (layer "B.Cu") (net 3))
 (segment (start 122.825 102.825) (end 123 103) (width 0.2) (layer "F.Cu") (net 8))
 (segment (start 122.825 101.5) (end 122.825 102.825) (width 0.2) (layer "F.Cu") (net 8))
 (segment (start 127.19 101.19) (end 127.19 98.5) (width 0.2) (layer "F.Cu") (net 8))
 (segment (start 128 102) (end 127.19 101.19) (width 0.2) (layer "F.Cu") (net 8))
 (via (at 123 103) (size 0.6) (drill 0.3) (layers "F.Cu" "B.Cu") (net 8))
 (via (at 128 102) (size 0.6) (drill 0.3) (layers "F.Cu" "B.Cu") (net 8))
 (segment (start 127 103) (end 128 102) (width 0.2) (layer "B.Cu") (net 8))
 (segment (start 123 103) (end 127 103) (width 0.2) (layer "B.Cu") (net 8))
 (segment (start 133.15 105.46) (end 134.69 107) (width 0.2) (layer "F.Cu") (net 5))
 (segment (start 133.15 104) (end 133.15 105.46) (width 0.2) (layer "F.Cu") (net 5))
 (segment (start 125.65 104.66) (end 125.65 104) (width 0.2) (layer "F.Cu") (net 7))
 (segment (start 123.31 107) (end 125.65 104.66) (width 0.2) (layer "F.Cu") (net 7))
 (segment (start 134.15 96) (end 134.15 97.46) (width 0.2) (layer "F.Cu") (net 6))
 (segment (start 134.15 97.46) (end 135.69 99) (width 0.2) (layer "F.Cu") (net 6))
 (segment (start 123.175 95.635) (end 121.31 97.5) (width 0.2) (layer "F.Cu") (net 2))
 (segment (start 123.175 94.5) (end 123.175 95.635) (width 0.2) (layer "F.Cu") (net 2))
 (segment (start 134.65 89.96) (end 135.69 91) (width 0.2) (layer "F.Cu") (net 4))
 (segment (start 134.65 87) (end 134.65 89.96) (width 0.2) (layer "F.Cu") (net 4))
 (segment (start 123.81 88.5) (end 123.81 90) (width 0.2) (layer "F.Cu") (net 9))
 (segment (start 124.175 88.135) (end 123.81 88.5) (width 0.2) (layer "F.Cu") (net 9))
 (segment (start 124.175 87.5) (end 124.175 88.135) (width 0.2) (layer "F.Cu") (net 9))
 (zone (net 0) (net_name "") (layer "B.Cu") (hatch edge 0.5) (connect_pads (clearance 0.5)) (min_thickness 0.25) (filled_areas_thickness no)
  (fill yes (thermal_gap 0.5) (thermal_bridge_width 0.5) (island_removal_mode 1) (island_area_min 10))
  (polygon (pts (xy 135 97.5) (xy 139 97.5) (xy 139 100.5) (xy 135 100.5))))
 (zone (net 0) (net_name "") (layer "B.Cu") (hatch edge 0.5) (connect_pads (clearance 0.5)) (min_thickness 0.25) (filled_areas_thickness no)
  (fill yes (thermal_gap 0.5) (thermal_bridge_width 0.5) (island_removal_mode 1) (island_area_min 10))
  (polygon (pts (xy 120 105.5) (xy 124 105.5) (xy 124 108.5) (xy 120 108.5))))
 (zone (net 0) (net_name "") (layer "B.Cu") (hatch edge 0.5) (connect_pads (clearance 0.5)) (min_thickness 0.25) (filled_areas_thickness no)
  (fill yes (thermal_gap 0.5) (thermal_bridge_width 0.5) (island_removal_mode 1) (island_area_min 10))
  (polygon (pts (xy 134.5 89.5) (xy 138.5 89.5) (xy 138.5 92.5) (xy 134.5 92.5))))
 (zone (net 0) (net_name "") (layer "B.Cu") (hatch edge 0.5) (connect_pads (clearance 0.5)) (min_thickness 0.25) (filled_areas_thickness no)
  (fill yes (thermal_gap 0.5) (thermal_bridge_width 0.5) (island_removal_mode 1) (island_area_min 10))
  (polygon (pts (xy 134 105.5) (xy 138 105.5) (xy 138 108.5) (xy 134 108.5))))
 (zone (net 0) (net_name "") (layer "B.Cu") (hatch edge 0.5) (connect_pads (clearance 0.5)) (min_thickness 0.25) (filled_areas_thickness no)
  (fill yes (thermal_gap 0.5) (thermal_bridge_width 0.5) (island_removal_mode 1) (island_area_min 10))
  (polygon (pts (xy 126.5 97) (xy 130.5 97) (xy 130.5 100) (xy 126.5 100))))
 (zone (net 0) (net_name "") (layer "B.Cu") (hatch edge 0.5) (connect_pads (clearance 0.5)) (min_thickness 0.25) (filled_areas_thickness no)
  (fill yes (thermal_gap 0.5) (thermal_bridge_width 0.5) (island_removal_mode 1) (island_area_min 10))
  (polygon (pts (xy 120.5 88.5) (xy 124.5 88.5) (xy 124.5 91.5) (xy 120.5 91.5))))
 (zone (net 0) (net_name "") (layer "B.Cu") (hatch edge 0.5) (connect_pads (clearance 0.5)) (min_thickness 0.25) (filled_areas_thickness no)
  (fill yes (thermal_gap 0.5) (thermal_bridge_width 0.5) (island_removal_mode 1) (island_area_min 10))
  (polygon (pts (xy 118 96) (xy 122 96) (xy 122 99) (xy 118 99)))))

